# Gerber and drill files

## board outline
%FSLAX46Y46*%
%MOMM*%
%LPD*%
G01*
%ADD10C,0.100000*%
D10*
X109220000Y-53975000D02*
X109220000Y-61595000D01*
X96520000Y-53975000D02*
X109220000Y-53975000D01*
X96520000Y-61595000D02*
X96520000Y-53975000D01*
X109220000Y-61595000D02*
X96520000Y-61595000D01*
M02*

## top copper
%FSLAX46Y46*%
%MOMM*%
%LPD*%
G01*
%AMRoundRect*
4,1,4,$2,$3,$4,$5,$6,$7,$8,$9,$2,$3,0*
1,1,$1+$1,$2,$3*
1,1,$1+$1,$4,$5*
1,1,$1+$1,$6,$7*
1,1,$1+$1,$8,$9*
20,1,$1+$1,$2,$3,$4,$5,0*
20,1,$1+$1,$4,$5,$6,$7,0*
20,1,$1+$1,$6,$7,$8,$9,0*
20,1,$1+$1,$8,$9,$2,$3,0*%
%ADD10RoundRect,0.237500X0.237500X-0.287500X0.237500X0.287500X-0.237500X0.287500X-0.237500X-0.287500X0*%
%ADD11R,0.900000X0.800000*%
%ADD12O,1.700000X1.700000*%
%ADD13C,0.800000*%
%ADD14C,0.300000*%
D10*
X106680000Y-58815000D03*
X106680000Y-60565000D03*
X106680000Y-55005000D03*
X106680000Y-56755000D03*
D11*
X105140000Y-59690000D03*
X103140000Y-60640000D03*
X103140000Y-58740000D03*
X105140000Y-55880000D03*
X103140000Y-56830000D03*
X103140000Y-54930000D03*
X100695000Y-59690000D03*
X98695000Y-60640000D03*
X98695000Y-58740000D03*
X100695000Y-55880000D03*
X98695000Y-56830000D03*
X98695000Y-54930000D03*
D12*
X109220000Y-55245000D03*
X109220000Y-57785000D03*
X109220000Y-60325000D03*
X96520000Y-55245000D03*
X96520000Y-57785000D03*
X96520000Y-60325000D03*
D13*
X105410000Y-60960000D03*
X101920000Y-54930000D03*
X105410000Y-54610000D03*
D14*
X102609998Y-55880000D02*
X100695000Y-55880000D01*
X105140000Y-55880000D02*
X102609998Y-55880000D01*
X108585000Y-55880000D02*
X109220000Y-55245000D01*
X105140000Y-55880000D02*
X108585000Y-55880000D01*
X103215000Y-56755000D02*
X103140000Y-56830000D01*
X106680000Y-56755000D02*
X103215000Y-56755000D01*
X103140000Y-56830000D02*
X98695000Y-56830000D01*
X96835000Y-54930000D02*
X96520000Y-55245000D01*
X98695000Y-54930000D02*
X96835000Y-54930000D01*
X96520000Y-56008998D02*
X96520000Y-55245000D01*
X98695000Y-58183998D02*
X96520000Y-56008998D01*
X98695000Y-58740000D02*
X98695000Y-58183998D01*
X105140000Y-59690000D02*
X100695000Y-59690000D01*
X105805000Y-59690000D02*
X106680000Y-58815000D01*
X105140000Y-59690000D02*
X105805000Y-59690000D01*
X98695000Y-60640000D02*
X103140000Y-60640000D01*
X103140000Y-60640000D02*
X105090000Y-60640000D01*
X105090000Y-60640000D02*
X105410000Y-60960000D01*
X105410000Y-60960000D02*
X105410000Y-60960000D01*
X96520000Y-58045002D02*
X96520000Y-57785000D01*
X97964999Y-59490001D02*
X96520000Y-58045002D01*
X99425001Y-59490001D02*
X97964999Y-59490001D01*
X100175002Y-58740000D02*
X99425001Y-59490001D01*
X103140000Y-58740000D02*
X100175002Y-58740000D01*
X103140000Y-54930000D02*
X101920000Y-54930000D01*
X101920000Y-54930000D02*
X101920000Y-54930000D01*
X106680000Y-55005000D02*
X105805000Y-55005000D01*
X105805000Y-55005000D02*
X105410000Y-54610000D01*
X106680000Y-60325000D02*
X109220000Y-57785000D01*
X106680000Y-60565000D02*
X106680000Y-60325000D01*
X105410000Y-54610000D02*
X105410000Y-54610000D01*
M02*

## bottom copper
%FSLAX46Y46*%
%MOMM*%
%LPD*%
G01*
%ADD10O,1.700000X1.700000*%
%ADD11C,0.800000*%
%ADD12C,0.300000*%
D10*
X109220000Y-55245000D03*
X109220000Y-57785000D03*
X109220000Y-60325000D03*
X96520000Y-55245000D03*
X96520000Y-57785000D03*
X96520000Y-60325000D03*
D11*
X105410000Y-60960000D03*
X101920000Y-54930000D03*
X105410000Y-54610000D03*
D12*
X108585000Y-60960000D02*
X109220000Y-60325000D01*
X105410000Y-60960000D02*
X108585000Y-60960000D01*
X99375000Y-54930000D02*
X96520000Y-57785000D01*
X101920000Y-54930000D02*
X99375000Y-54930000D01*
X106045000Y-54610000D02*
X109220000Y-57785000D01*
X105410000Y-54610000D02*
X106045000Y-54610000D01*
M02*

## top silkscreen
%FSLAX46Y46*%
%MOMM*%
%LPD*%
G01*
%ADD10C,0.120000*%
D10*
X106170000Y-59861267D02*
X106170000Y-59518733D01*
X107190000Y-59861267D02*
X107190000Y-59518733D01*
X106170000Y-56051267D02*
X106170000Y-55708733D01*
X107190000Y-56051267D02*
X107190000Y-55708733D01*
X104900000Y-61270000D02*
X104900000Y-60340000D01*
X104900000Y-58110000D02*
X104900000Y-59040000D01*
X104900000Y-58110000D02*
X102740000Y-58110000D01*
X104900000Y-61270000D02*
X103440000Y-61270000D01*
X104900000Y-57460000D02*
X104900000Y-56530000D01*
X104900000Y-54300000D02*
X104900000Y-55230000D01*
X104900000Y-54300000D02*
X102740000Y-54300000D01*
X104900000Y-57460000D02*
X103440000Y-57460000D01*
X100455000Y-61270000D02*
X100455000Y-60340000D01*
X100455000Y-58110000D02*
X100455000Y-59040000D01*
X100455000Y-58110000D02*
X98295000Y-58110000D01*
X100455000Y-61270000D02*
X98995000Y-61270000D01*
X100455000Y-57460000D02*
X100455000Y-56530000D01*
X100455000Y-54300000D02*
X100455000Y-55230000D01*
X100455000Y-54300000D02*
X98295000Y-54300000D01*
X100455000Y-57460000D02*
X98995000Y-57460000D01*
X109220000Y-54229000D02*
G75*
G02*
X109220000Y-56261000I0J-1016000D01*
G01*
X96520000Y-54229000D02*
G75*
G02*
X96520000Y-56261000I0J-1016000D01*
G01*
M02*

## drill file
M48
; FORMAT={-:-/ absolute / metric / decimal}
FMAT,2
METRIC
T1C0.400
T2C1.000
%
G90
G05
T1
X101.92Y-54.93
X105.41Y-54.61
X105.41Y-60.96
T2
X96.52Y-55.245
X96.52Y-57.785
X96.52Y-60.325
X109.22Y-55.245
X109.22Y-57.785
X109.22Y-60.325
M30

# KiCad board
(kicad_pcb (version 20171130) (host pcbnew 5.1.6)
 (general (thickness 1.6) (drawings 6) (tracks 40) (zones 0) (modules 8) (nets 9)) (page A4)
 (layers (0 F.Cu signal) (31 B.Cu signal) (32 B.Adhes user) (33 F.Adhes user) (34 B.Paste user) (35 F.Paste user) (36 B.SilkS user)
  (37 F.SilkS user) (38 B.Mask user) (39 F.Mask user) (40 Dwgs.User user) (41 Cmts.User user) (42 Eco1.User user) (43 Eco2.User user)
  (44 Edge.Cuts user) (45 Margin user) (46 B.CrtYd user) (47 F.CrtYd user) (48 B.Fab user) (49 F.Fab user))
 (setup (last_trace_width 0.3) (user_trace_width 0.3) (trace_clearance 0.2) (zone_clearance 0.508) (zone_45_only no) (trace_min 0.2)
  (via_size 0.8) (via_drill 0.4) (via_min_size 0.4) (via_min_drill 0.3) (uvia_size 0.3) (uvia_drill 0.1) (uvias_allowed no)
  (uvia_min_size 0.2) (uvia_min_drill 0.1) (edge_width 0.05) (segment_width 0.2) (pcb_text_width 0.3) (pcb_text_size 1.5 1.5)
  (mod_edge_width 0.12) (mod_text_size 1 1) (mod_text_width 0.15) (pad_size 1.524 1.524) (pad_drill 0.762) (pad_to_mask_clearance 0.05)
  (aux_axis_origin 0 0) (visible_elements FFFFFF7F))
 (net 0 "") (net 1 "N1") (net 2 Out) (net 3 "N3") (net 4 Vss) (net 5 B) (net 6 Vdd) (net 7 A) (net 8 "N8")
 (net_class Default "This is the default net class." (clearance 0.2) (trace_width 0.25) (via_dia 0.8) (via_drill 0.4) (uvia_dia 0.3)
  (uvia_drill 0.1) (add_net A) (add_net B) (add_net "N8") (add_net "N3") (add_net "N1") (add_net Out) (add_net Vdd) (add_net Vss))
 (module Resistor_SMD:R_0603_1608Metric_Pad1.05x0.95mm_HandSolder (layer F.Cu) (at 106.68 59.69 90)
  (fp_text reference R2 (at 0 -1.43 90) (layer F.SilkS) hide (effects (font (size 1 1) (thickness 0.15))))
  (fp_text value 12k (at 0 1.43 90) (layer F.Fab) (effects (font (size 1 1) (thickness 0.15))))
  (fp_line (start -0.171267 -0.51) (end 0.171267 -0.51) (layer F.SilkS) (width 0.12))
  (fp_line (start -0.171267 0.51) (end 0.171267 0.51) (layer F.SilkS) (width 0.12))
  (pad 2 smd roundrect (at 0.875 0 90) (size 1.05 0.95) (layers F.Cu F.Paste F.Mask) (roundrect_rratio 0.25) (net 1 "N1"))
  (pad 1 smd roundrect (at -0.875 0 90) (size 1.05 0.95) (layers F.Cu F.Paste F.Mask) (roundrect_rratio 0.25) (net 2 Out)))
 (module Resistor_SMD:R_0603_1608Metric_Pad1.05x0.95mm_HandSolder (layer F.Cu) (at 106.68 55.88 90)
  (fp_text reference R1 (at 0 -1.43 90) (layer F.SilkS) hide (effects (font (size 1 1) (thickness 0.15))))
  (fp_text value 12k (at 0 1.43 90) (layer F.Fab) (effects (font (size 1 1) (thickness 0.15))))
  (fp_line (start -0.171267 -0.51) (end 0.171267 -0.51) (layer F.SilkS) (width 0.12))
  (fp_line (start -0.171267 0.51) (end 0.171267 0.51) (layer F.SilkS) (width 0.12))
  (pad 2 smd roundrect (at 0.875 0 90) (size 1.05 0.95) (layers F.Cu F.Paste F.Mask) (roundrect_rratio 0.25) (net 2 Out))
  (pad 1 smd roundrect (at -0.875 0 90) (size 1.05 0.95) (layers F.Cu F.Paste F.Mask) (roundrect_rratio 0.25) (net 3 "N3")))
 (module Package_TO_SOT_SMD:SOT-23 (layer F.Cu) (at 104.14 59.69)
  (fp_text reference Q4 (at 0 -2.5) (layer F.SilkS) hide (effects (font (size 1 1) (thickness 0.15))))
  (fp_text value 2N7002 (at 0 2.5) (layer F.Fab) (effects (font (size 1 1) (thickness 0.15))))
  (fp_line (start 0.76 1.58) (end 0.76 0.65) (layer F.SilkS) (width 0.12))
  (fp_line (start 0.76 -1.58) (end 0.76 -0.65) (layer F.SilkS) (width 0.12))
  (fp_line (start 0.76 -1.58) (end -1.4 -1.58) (layer F.SilkS) (width 0.12))
  (fp_line (start 0.76 1.58) (end -0.7 1.58) (layer F.SilkS) (width 0.12))
  (pad 3 smd rect (at 1 0) (size 0.9 0.8) (layers F.Cu F.Paste F.Mask) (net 1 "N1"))
  (pad 2 smd rect (at -1 0.95) (size 0.9 0.8) (layers F.Cu F.Paste F.Mask) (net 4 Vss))
  (pad 1 smd rect (at -1 -0.95) (size 0.9 0.8) (layers F.Cu F.Paste F.Mask) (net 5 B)))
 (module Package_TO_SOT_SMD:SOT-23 (layer F.Cu) (at 104.14 55.88)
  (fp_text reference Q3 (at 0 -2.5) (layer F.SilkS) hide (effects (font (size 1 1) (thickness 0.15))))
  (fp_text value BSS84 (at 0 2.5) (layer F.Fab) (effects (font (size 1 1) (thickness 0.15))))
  (fp_line (start 0.76 1.58) (end 0.76 0.65) (layer F.SilkS) (width 0.12))
  (fp_line (start 0.76 -1.58) (end 0.76 -0.65) (layer F.SilkS) (width 0.12))
  (fp_line (start 0.76 -1.58) (end -1.4 -1.58) (layer F.SilkS) (width 0.12))
  (fp_line (start 0.76 1.58) (end -0.7 1.58) (layer F.SilkS) (width 0.12))
  (pad 3 smd rect (at 1 0) (size 0.9 0.8) (layers F.Cu F.Paste F.Mask) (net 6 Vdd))
  (pad 2 smd rect (at -1 0.95) (size 0.9 0.8) (layers F.Cu F.Paste F.Mask) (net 3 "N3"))
  (pad 1 smd rect (at -1 -0.95) (size 0.9 0.8) (layers F.Cu F.Paste F.Mask) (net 5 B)))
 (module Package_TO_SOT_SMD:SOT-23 (layer F.Cu) (at 99.695 59.69)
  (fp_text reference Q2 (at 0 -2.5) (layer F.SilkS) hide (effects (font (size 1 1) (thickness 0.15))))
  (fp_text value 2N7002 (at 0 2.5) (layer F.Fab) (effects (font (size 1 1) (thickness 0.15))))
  (fp_line (start 0.76 1.58) (end 0.76 0.65) (layer F.SilkS) (width 0.12))
  (fp_line (start 0.76 -1.58) (end 0.76 -0.65) (layer F.SilkS) (width 0.12))
  (fp_line (start 0.76 -1.58) (end -1.4 -1.58) (layer F.SilkS) (width 0.12))
  (fp_line (start 0.76 1.58) (end -0.7 1.58) (layer F.SilkS) (width 0.12))
  (pad 3 smd rect (at 1 0) (size 0.9 0.8) (layers F.Cu F.Paste F.Mask) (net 1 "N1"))
  (pad 2 smd rect (at -1 0.95) (size 0.9 0.8) (layers F.Cu F.Paste F.Mask) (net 4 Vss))
  (pad 1 smd rect (at -1 -0.95) (size 0.9 0.8) (layers F.Cu F.Paste F.Mask) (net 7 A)))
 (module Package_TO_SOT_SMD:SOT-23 (layer F.Cu) (at 99.695 55.88)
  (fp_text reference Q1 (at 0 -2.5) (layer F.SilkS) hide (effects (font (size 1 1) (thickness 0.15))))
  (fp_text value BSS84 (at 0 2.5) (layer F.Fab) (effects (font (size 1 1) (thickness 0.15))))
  (fp_line (start 0.76 1.58) (end 0.76 0.65) (layer F.SilkS) (width 0.12))
  (fp_line (start 0.76 -1.58) (end 0.76 -0.65) (layer F.SilkS) (width 0.12))
  (fp_line (start 0.76 -1.58) (end -1.4 -1.58) (layer F.SilkS) (width 0.12))
  (fp_line (start 0.76 1.58) (end -0.7 1.58) (layer F.SilkS) (width 0.12))
  (pad 3 smd rect (at 1 0) (size 0.9 0.8) (layers F.Cu F.Paste F.Mask) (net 6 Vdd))
  (pad 2 smd rect (at -1 0.95) (size 0.9 0.8) (layers F.Cu F.Paste F.Mask) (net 3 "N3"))
  (pad 1 smd rect (at -1 -0.95) (size 0.9 0.8) (layers F.Cu F.Paste F.Mask) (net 7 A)))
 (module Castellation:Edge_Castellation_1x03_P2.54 (layer F.Cu) (at 109.22 55.245)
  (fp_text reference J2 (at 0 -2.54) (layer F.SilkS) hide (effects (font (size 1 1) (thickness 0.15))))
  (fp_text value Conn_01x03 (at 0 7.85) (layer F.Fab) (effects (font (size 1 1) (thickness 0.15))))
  (fp_arc (start 0 0) (end 0 1.016) (angle -180) (layer F.SilkS) (width 0.12))
  (pad 1 thru_hole oval (at 0 0) (size 1.7 1.7) (drill 1) (layers *.Cu *.Mask) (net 6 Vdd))
  (pad 2 thru_hole oval (at 0 2.54) (size 1.7 1.7) (drill 1) (layers *.Cu *.Mask) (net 2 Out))
  (pad 3 thru_hole oval (at 0 5.08) (size 1.7 1.7) (drill 1) (layers *.Cu *.Mask) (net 4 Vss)))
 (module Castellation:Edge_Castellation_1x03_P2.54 (layer F.Cu) (at 96.52 55.245)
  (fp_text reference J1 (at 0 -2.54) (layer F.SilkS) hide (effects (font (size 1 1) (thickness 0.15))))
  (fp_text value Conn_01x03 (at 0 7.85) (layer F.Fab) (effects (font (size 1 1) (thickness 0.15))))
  (fp_arc (start 0 0) (end 0 1.016) (angle -180) (layer F.SilkS) (width 0.12))
  (pad 1 thru_hole oval (at 0 0) (size 1.7 1.7) (drill 1) (layers *.Cu *.Mask) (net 7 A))
  (pad 2 thru_hole oval (at 0 2.54) (size 1.7 1.7) (drill 1) (layers *.Cu *.Mask) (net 5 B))
  (pad 3 thru_hole oval (at 0 5.08) (size 1.7 1.7) (drill 1) (layers *.Cu *.Mask) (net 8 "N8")))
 (gr_line (start 109.22 53.975) (end 109.22 61.595) (layer Edge.Cuts) (width 0.1))
 (gr_line (start 96.52 53.975) (end 109.22 53.975) (layer Edge.Cuts) (width 0.1))
 (gr_line (start 96.52 61.595) (end 96.52 53.975) (layer Edge.Cuts) (width 0.1))
 (gr_line (start 109.22 61.595) (end 96.52 61.595) (layer Edge.Cuts) (width 0.1))
 (segment (start 102.609998 55.88) (end 100.695 55.88) (width 0.3) (layer F.Cu) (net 6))
 (segment (start 105.14 55.88) (end 102.609998 55.88) (width 0.3) (layer F.Cu) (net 6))
 (segment (start 108.585 55.88) (end 109.22 55.245) (width 0.3) (layer F.Cu) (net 6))
 (segment (start 105.14 55.88) (end 108.585 55.88) (width 0.3) (layer F.Cu) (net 6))
 (segment (start 103.215 56.755) (end 103.14 56.83) (width 0.3) (layer F.Cu) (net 3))
 (segment (start 106.68 56.755) (end 103.215 56.755) (width 0.3) (layer F.Cu) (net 3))
 (segment (start 103.14 56.83) (end 98.695 56.83) (width 0.3) (layer F.Cu) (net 3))
 (segment (start 96.835 54.93) (end 96.52 55.245) (width 0.3) (layer F.Cu) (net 7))
 (segment (start 98.695 54.93) (end 96.835 54.93) (width 0.3) (layer F.Cu) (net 7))
 (segment (start 96.52 56.008998) (end 96.52 55.245) (width 0.3) (layer F.Cu) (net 7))
 (segment (start 98.695 58.183998) (end 96.52 56.008998) (width 0.3) (layer F.Cu) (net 7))
 (segment (start 98.695 58.74) (end 98.695 58.183998) (width 0.3) (layer F.Cu) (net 7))
 (segment (start 105.14 59.69) (end 100.695 59.69) (width 0.3) (layer F.Cu) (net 1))
 (segment (start 105.805 59.69) (end 106.68 58.815) (width 0.3) (layer F.Cu) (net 1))
 (segment (start 105.14 59.69) (end 105.805 59.69) (width 0.3) (layer F.Cu) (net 1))
 (segment (start 98.695 60.64) (end 103.14 60.64) (width 0.3) (layer F.Cu) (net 4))
 (segment (start 103.14 60.64) (end 105.09 60.64) (width 0.3) (layer F.Cu) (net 4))
 (segment (start 105.09 60.64) (end 105.41 60.96) (width 0.3) (layer F.Cu) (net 4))
 (segment (start 105.41 60.96) (end 105.41 60.96) (width 0.3) (layer F.Cu) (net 4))
 (via (at 105.41 60.96) (size 0.8) (drill 0.4) (layers F.Cu B.Cu) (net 4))
 (segment (start 108.585 60.96) (end 109.22 60.325) (width 0.3) (layer B.Cu) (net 4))
 (segment (start 105.41 60.96) (end 108.585 60.96) (width 0.3) (layer B.Cu) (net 4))
 (segment (start 96.52 58.045002) (end 96.52 57.785) (width 0.3) (layer F.Cu) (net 5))
 (segment (start 97.964999 59.490001) (end 96.52 58.045002) (width 0.3) (layer F.Cu) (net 5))
 (segment (start 99.425001 59.490001) (end 97.964999 59.490001) (width 0.3) (layer F.Cu) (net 5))
 (segment (start 100.175002 58.74) (end 99.425001 59.490001) (width 0.3) (layer F.Cu) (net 5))
 (segment (start 103.14 58.74) (end 100.175002 58.74) (width 0.3) (layer F.Cu) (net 5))
 (segment (start 103.14 54.93) (end 101.92 54.93) (width 0.3) (layer F.Cu) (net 5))
 (segment (start 101.92 54.93) (end 101.92 54.93) (width 0.3) (layer F.Cu) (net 5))
 (via (at 101.92 54.93) (size 0.8) (drill 0.4) (layers F.Cu B.Cu) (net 5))
 (segment (start 99.375 54.93) (end 96.52 57.785) (width 0.3) (layer B.Cu) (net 5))
 (segment (start 101.92 54.93) (end 99.375 54.93) (width 0.3) (layer B.Cu) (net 5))
 (segment (start 106.68 55.005) (end 105.805 55.005) (width 0.3) (layer F.Cu) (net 2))
 (segment (start 105.805 55.005) (end 105.41 54.61) (width 0.3) (layer F.Cu) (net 2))
 (segment (start 106.68 60.325) (end 109.22 57.785) (width 0.3) (layer F.Cu) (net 2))
 (segment (start 106.68 60.565) (end 106.68 60.325) (width 0.3) (layer F.Cu) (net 2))
 (segment (start 105.41 54.61) (end 105.41 54.61) (width 0.3) (layer F.Cu) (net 2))
 (via (at 105.41 54.61) (size 0.8) (drill 0.4) (layers F.Cu B.Cu) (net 2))
 (segment (start 106.045 54.61) (end 109.22 57.785) (width 0.3) (layer B.Cu) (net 2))
 (segment (start 105.41 54.61) (end 106.045 54.61) (width 0.3) (layer B.Cu) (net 2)))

